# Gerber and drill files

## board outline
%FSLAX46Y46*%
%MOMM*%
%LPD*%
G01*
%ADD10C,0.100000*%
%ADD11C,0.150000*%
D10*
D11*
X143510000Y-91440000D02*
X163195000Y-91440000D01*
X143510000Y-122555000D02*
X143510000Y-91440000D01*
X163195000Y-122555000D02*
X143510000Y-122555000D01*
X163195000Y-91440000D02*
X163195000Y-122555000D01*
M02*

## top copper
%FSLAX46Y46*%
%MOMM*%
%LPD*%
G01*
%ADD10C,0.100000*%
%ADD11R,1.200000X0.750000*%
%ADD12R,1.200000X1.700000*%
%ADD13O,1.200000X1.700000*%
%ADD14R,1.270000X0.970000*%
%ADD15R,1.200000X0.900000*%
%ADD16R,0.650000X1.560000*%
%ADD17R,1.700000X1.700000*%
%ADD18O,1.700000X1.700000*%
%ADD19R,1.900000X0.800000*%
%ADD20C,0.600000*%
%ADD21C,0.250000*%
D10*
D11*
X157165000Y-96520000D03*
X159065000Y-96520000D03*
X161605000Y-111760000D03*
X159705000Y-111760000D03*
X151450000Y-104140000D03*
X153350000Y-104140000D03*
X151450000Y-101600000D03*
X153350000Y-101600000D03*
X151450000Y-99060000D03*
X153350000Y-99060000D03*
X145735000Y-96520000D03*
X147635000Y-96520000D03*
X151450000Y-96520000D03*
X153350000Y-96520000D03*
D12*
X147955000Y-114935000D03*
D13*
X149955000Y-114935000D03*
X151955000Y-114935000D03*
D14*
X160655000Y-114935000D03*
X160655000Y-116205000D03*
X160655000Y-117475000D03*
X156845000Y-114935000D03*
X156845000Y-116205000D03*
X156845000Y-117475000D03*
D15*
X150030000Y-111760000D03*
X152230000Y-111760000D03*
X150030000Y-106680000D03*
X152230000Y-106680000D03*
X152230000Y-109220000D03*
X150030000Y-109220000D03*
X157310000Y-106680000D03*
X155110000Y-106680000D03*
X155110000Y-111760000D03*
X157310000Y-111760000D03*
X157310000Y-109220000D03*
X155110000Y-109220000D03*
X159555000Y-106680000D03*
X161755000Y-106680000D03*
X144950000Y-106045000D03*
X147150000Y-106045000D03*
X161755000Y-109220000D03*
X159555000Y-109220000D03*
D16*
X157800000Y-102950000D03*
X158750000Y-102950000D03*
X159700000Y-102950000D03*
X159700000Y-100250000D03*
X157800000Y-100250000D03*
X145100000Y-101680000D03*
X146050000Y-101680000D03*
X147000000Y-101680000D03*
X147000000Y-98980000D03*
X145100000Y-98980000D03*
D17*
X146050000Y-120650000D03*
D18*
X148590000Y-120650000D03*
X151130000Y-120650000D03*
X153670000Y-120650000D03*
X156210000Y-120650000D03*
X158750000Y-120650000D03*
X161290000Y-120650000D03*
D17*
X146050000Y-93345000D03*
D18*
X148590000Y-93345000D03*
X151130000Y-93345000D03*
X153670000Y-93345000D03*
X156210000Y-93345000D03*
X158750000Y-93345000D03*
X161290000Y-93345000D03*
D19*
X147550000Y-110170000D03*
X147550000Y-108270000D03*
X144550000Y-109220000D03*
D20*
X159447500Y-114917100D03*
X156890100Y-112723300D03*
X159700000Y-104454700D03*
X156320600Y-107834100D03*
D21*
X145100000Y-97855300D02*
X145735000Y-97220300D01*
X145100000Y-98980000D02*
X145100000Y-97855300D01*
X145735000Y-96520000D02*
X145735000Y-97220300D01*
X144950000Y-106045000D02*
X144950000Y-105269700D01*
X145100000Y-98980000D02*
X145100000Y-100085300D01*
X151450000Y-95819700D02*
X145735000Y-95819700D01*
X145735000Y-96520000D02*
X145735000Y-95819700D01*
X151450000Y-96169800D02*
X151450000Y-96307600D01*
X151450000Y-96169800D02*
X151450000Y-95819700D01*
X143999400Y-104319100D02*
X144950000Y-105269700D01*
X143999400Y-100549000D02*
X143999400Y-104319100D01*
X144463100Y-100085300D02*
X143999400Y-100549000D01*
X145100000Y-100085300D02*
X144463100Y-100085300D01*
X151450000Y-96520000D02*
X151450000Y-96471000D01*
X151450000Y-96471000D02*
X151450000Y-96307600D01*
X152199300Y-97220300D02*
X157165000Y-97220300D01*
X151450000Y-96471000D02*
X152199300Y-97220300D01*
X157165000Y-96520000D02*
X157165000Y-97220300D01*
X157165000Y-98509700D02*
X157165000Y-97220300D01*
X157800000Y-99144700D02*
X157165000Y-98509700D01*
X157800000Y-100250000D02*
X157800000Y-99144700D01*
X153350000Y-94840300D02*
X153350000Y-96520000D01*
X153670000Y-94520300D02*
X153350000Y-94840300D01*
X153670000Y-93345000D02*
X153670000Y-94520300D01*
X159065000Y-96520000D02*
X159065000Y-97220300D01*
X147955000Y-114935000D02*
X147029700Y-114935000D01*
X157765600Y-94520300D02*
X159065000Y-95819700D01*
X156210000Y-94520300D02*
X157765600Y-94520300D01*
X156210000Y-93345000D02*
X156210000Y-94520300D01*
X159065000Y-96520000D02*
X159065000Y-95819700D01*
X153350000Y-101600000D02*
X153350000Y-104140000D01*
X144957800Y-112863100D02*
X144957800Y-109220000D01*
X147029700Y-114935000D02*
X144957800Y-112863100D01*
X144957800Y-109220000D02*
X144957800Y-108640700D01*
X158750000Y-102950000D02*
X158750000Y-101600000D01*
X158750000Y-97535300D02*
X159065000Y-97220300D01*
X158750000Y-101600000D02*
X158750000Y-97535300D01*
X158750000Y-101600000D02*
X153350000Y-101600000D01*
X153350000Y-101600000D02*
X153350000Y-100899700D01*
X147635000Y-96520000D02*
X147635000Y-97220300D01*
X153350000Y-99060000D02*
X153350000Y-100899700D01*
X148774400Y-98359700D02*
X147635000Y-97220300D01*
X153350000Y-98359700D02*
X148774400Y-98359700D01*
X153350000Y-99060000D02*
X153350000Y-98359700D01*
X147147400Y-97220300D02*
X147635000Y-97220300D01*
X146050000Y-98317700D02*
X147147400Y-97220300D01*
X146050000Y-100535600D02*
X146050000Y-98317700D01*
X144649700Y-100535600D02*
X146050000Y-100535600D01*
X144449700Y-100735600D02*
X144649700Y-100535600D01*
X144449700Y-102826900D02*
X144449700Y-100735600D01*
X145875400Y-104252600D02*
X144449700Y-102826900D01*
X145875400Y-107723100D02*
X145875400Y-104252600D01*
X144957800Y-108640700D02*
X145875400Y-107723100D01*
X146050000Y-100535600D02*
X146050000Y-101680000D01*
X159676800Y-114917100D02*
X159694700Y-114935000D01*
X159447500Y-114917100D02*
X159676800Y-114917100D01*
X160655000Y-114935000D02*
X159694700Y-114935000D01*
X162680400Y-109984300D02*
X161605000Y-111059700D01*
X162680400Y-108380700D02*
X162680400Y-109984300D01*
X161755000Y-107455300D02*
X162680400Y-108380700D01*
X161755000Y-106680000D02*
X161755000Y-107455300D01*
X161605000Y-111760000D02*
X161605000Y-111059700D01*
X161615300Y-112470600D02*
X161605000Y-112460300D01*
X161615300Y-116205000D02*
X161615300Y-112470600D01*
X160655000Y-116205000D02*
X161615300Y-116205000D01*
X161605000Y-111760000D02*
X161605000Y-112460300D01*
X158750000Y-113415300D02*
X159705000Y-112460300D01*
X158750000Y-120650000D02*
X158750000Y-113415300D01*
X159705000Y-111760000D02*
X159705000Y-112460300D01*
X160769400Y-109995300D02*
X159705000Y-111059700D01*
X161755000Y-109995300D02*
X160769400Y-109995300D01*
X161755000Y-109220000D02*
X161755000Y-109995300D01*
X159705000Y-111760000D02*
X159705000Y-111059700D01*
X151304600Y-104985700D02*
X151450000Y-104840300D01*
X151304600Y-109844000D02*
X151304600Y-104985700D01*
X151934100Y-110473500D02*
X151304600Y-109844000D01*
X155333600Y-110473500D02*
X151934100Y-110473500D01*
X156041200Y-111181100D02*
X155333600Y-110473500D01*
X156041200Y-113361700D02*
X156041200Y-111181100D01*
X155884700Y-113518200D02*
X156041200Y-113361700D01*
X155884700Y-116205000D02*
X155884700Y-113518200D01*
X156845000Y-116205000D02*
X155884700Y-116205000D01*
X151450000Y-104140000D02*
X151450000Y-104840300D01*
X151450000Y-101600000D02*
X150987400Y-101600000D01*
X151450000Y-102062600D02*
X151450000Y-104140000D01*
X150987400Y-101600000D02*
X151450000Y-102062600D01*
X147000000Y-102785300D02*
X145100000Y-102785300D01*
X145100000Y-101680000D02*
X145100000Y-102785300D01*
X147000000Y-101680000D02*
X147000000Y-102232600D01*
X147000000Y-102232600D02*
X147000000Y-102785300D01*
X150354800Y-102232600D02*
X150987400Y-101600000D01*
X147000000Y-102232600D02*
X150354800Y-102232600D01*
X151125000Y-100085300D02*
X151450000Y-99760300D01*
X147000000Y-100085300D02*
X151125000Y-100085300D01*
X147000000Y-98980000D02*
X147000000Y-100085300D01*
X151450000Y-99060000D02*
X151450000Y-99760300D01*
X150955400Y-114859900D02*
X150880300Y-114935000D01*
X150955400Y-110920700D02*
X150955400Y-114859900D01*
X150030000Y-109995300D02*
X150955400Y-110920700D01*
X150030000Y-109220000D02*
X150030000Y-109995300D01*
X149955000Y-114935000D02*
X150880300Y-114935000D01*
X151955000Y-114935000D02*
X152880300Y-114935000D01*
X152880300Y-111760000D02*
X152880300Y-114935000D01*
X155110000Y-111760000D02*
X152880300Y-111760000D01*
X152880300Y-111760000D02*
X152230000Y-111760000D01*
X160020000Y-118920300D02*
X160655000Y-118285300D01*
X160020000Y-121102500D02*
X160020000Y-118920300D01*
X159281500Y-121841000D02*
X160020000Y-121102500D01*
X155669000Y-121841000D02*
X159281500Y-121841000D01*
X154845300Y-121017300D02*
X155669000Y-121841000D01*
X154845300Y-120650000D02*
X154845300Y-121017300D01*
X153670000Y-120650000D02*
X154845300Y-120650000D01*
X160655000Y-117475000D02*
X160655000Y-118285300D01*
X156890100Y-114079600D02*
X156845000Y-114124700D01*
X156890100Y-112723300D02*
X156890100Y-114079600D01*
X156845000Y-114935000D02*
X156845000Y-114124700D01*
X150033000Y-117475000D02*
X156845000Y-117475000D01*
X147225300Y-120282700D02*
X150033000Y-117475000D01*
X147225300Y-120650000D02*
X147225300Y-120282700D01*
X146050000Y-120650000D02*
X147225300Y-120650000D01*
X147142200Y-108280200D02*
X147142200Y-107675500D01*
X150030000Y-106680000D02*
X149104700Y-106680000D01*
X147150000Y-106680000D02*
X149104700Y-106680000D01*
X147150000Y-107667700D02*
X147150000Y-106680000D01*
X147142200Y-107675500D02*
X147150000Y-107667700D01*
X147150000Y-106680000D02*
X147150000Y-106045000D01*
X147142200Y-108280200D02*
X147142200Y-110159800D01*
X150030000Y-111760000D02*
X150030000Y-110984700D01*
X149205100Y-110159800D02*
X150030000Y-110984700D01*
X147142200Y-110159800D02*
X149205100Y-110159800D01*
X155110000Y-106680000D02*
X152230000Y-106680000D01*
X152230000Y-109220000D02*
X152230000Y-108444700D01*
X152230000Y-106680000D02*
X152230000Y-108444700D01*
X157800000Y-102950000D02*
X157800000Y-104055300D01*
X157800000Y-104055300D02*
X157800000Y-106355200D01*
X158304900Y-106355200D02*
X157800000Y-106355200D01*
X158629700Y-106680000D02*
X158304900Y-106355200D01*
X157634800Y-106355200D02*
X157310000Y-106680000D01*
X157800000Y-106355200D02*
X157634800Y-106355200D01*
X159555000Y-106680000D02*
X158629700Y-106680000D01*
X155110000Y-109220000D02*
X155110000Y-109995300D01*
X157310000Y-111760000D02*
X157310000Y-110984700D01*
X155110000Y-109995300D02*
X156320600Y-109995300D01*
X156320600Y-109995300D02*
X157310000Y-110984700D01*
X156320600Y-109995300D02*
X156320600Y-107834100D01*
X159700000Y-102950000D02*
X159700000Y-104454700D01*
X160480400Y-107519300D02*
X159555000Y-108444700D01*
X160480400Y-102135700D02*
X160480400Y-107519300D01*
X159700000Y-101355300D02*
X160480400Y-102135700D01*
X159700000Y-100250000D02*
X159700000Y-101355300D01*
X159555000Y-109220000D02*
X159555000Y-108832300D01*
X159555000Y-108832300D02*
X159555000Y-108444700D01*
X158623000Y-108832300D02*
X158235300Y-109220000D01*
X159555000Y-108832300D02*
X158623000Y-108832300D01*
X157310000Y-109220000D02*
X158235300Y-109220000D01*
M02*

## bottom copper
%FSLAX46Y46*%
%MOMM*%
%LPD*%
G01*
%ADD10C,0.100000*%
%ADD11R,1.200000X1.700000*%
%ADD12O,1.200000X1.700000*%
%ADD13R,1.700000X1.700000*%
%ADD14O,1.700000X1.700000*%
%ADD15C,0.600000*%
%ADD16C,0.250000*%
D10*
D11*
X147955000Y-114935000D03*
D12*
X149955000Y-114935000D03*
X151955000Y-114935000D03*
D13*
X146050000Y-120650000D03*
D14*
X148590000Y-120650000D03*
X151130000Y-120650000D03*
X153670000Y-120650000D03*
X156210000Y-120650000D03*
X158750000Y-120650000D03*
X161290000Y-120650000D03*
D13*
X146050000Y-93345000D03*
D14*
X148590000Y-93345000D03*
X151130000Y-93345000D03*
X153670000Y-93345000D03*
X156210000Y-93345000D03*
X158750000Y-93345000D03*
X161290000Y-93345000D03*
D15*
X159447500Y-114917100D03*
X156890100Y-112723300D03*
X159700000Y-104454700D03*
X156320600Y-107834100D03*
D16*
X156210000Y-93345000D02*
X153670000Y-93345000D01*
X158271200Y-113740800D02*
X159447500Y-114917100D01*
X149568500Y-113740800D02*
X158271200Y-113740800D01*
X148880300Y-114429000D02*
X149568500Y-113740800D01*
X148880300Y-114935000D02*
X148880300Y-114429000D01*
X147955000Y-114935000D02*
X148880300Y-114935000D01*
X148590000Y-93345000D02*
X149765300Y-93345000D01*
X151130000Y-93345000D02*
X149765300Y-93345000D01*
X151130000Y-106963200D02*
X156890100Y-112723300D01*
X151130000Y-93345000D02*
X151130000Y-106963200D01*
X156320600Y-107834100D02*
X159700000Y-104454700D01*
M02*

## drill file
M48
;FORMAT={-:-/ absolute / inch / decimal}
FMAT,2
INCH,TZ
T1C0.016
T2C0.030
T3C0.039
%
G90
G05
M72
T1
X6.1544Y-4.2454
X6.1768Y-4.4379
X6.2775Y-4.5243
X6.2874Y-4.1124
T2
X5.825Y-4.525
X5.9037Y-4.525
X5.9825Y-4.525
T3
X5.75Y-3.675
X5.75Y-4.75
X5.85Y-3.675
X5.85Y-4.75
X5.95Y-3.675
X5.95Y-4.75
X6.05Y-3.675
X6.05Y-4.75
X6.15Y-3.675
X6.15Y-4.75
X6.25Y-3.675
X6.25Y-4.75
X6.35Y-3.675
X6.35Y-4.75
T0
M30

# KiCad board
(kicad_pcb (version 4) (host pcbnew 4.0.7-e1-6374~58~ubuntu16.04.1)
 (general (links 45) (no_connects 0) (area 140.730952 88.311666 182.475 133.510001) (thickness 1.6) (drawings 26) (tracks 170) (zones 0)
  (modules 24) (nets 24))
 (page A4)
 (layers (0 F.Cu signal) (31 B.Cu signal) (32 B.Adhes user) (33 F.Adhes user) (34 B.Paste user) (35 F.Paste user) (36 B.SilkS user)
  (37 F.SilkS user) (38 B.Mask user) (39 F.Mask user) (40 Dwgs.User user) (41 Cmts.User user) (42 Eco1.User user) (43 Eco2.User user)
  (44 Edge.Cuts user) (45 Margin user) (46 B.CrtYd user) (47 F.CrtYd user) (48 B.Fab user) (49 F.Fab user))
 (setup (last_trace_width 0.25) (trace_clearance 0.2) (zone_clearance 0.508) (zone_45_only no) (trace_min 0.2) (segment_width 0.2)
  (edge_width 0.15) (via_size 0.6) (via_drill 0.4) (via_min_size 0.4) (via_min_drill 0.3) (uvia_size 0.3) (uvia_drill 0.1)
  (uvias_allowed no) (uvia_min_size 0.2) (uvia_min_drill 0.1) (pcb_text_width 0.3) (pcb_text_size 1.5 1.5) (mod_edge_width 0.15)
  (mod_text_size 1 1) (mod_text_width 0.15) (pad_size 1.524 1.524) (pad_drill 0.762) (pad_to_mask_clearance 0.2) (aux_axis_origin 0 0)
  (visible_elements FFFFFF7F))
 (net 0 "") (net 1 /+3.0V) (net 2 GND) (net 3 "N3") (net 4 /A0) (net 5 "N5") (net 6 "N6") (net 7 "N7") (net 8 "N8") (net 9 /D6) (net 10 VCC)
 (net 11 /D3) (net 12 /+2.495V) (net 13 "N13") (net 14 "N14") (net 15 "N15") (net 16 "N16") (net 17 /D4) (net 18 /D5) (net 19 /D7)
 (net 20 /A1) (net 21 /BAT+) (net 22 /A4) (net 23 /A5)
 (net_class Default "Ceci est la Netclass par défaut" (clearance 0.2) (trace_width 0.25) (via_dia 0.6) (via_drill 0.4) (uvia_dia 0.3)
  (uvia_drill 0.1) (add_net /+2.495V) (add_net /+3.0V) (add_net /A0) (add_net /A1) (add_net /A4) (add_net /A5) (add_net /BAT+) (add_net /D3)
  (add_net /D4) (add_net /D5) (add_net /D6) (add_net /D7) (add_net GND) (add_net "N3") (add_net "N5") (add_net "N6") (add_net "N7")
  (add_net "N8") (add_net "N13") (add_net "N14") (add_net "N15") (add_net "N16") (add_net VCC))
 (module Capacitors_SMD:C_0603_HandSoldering (layer F.Cu) (at 158.115 96.52)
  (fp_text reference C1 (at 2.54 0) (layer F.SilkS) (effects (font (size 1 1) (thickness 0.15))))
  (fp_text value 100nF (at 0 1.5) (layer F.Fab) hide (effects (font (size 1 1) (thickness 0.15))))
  (pad 1 smd rect (at -0.95 0) (size 1.2 0.75) (layers F.Cu F.Paste F.Mask) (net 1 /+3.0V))
  (pad 2 smd rect (at 0.95 0) (size 1.2 0.75) (layers F.Cu F.Paste F.Mask) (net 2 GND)))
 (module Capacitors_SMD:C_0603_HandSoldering (layer F.Cu) (at 160.655 111.76 180)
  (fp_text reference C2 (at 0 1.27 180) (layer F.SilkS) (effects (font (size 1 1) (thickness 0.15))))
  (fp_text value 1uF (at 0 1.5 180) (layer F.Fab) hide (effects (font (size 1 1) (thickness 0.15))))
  (pad 1 smd rect (at -0.95 0 180) (size 1.2 0.75) (layers F.Cu F.Paste F.Mask) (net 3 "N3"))
  (pad 2 smd rect (at 0.95 0 180) (size 1.2 0.75) (layers F.Cu F.Paste F.Mask) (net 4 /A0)))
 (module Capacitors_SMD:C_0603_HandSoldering (layer F.Cu) (at 152.4 104.14)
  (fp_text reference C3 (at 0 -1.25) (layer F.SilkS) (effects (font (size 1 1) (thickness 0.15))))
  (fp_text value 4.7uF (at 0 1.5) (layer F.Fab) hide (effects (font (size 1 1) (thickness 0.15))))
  (pad 1 smd rect (at -0.95 0) (size 1.2 0.75) (layers F.Cu F.Paste F.Mask) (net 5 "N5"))
  (pad 2 smd rect (at 0.95 0) (size 1.2 0.75) (layers F.Cu F.Paste F.Mask) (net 2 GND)))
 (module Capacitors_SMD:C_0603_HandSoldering (layer F.Cu) (at 152.4 101.6)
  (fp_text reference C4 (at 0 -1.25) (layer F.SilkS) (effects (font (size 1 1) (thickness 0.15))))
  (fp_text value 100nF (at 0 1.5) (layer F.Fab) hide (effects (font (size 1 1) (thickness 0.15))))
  (pad 1 smd rect (at -0.95 0) (size 1.2 0.75) (layers F.Cu F.Paste F.Mask) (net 5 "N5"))
  (pad 2 smd rect (at 0.95 0) (size 1.2 0.75) (layers F.Cu F.Paste F.Mask) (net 2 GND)))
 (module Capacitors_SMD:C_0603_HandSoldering (layer F.Cu) (at 152.4 99.06)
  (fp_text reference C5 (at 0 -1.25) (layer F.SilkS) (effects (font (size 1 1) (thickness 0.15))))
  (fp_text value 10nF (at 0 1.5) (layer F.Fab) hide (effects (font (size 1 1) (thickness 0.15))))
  (pad 1 smd rect (at -0.95 0) (size 1.2 0.75) (layers F.Cu F.Paste F.Mask) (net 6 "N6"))
  (pad 2 smd rect (at 0.95 0) (size 1.2 0.75) (layers F.Cu F.Paste F.Mask) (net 2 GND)))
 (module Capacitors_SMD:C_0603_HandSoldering (layer F.Cu) (at 146.685 96.52)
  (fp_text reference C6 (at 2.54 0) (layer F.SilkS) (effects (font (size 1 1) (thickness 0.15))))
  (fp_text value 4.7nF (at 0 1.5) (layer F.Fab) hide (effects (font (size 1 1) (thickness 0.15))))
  (pad 1 smd rect (at -0.95 0) (size 1.2 0.75) (layers F.Cu F.Paste F.Mask) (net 1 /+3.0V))
  (pad 2 smd rect (at 0.95 0) (size 1.2 0.75) (layers F.Cu F.Paste F.Mask) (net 2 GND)))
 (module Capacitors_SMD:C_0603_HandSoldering (layer F.Cu) (at 152.4 96.52)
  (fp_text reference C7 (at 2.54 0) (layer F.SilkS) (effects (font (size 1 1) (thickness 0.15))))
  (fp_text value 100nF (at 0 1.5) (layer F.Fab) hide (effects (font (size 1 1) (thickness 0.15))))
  (pad 1 smd rect (at -0.95 0) (size 1.2 0.75) (layers F.Cu F.Paste F.Mask) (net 1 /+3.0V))
  (pad 2 smd rect (at 0.95 0) (size 1.2 0.75) (layers F.Cu F.Paste F.Mask) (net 2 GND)))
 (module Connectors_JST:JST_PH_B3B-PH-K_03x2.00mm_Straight (layer F.Cu) (at 147.955 114.935)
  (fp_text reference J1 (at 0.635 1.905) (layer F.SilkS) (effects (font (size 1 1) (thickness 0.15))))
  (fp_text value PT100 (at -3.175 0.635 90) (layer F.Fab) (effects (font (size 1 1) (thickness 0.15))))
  (pad 1 thru_hole rect (at 0 0) (size 1.2 1.7) (drill 0.75) (layers *.Cu *.Mask) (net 2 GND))
  (pad 2 thru_hole oval (at 2 0) (size 1.2 1.7) (drill 0.75) (layers *.Cu *.Mask) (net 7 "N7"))
  (pad 3 thru_hole oval (at 4 0) (size 1.2 1.7) (drill 0.75) (layers *.Cu *.Mask) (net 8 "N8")))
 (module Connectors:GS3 (layer F.Cu) (at 160.655 116.205)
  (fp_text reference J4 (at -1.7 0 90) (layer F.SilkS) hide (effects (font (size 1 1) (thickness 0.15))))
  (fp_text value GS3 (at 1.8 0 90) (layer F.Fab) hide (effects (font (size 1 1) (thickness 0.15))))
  (pad 1 smd rect (at 0 -1.27) (size 1.27 0.97) (layers F.Cu F.Paste F.Mask) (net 2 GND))
  (pad 2 smd rect (at 0 0) (size 1.27 0.97) (layers F.Cu F.Paste F.Mask) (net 3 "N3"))
  (pad 3 smd rect (at 0 1.27) (size 1.27 0.97) (layers F.Cu F.Paste F.Mask) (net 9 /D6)))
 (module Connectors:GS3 (layer F.Cu) (at 156.845 116.205)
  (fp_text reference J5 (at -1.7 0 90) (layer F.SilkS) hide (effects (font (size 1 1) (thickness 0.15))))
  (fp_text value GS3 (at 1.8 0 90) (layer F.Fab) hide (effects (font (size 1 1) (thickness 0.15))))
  (pad 1 smd rect (at 0 -1.27) (size 1.27 0.97) (layers F.Cu F.Paste F.Mask) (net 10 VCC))
  (pad 2 smd rect (at 0 0) (size 1.27 0.97) (layers F.Cu F.Paste F.Mask) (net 5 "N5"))
  (pad 3 smd rect (at 0 1.27) (size 1.27 0.97) (layers F.Cu F.Paste F.Mask) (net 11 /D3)))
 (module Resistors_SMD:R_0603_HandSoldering (layer F.Cu) (at 151.13 111.76)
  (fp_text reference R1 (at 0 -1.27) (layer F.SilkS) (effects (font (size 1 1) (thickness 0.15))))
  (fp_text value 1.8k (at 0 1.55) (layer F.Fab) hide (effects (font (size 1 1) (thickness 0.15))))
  (pad 1 smd rect (at -1.1 0) (size 1.2 0.9) (layers F.Cu F.Paste F.Mask) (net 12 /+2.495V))
  (pad 2 smd rect (at 1.1 0) (size 1.2 0.9) (layers F.Cu F.Paste F.Mask) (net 8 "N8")))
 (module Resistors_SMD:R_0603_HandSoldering (layer F.Cu) (at 151.13 106.68)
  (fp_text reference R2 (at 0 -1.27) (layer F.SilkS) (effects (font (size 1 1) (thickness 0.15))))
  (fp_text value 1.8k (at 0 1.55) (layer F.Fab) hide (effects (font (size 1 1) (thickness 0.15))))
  (pad 1 smd rect (at -1.1 0) (size 1.2 0.9) (layers F.Cu F.Paste F.Mask) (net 12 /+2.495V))
  (pad 2 smd rect (at 1.1 0) (size 1.2 0.9) (layers F.Cu F.Paste F.Mask) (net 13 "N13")))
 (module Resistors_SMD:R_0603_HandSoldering (layer F.Cu) (at 151.13 109.22 180)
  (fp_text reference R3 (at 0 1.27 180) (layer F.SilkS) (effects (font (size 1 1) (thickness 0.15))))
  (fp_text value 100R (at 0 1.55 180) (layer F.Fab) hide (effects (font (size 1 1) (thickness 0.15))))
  (pad 1 smd rect (at -1.1 0 180) (size 1.2 0.9) (layers F.Cu F.Paste F.Mask) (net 13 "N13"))
  (pad 2 smd rect (at 1.1 0 180) (size 1.2 0.9) (layers F.Cu F.Paste F.Mask) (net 7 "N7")))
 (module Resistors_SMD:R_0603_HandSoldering (layer F.Cu) (at 156.21 106.68 180)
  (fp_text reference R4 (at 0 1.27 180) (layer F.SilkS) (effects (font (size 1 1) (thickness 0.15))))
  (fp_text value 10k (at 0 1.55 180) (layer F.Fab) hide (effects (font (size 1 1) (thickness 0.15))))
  (pad 1 smd rect (at -1.1 0 180) (size 1.2 0.9) (layers F.Cu F.Paste F.Mask) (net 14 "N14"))
  (pad 2 smd rect (at 1.1 0 180) (size 1.2 0.9) (layers F.Cu F.Paste F.Mask) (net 13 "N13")))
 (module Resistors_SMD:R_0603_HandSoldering (layer F.Cu) (at 156.21 111.76)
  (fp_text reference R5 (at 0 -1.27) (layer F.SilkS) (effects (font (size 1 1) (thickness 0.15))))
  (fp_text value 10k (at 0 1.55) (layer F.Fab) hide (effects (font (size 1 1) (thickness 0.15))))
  (pad 1 smd rect (at -1.1 0) (size 1.2 0.9) (layers F.Cu F.Paste F.Mask) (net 8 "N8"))
  (pad 2 smd rect (at 1.1 0) (size 1.2 0.9) (layers F.Cu F.Paste F.Mask) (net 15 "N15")))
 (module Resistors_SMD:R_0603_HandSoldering (layer F.Cu) (at 156.21 109.22 180)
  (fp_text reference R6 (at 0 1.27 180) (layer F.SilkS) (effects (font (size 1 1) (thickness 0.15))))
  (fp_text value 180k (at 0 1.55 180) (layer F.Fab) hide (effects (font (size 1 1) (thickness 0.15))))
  (pad 1 smd rect (at -1.1 0 180) (size 1.2 0.9) (layers F.Cu F.Paste F.Mask) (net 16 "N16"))
  (pad 2 smd rect (at 1.1 0 180) (size 1.2 0.9) (layers F.Cu F.Paste F.Mask) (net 15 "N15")))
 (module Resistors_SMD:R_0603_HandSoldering (layer F.Cu) (at 160.655 106.68)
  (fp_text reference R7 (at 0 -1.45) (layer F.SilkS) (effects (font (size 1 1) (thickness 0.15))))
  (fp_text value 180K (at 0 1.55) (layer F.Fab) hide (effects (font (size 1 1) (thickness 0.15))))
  (pad 1 smd rect (at -1.1 0) (size 1.2 0.9) (layers F.Cu F.Paste F.Mask) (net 14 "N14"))
  (pad 2 smd rect (at 1.1 0) (size 1.2 0.9) (layers F.Cu F.Paste F.Mask) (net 3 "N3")))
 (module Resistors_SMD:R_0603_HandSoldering (layer F.Cu) (at 146.05 106.045)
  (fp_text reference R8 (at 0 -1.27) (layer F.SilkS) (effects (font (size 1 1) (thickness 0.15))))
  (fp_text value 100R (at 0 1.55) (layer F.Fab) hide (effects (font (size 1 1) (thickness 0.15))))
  (pad 1 smd rect (at -1.1 0) (size 1.2 0.9) (layers F.Cu F.Paste F.Mask) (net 1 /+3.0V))
  (pad 2 smd rect (at 1.1 0) (size 1.2 0.9) (layers F.Cu F.Paste F.Mask) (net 12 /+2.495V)))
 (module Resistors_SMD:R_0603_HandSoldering (layer F.Cu) (at 160.655 109.22 180)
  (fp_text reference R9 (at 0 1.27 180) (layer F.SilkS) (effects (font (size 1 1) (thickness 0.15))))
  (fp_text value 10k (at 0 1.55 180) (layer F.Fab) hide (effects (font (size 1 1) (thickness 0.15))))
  (pad 1 smd rect (at -1.1 0 180) (size 1.2 0.9) (layers F.Cu F.Paste F.Mask) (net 4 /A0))
  (pad 2 smd rect (at 1.1 0 180) (size 1.2 0.9) (layers F.Cu F.Paste F.Mask) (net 16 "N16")))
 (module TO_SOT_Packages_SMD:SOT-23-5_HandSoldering (layer F.Cu) (at 158.75 101.6 90)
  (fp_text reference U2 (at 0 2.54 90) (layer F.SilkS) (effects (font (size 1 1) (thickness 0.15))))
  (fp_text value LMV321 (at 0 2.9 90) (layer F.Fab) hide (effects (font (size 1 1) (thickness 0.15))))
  (pad 1 smd rect (at -1.35 -0.95 90) (size 1.56 0.65) (layers F.Cu F.Paste F.Mask) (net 14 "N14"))
  (pad 2 smd rect (at -1.35 0 90) (size 1.56 0.65) (layers F.Cu F.Paste F.Mask) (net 2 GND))
  (pad 3 smd rect (at -1.35 0.95 90) (size 1.56 0.65) (layers F.Cu F.Paste F.Mask) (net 15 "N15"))
  (pad 4 smd rect (at 1.35 0.95 90) (size 1.56 0.65) (layers F.Cu F.Paste F.Mask) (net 16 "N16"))
  (pad 5 smd rect (at 1.35 -0.95 90) (size 1.56 0.65) (layers F.Cu F.Paste F.Mask) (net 1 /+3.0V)))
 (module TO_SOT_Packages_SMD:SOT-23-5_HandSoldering (layer F.Cu) (at 146.05 100.33 90)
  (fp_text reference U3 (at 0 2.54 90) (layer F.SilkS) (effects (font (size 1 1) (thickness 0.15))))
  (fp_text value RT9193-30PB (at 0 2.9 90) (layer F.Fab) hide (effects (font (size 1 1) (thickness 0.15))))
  (pad 1 smd rect (at -1.35 -0.95 90) (size 1.56 0.65) (layers F.Cu F.Paste F.Mask) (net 5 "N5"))
  (pad 2 smd rect (at -1.35 0 90) (size 1.56 0.65) (layers F.Cu F.Paste F.Mask) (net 2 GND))
  (pad 3 smd rect (at -1.35 0.95 90) (size 1.56 0.65) (layers F.Cu F.Paste F.Mask) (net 5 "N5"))
  (pad 4 smd rect (at 1.35 0.95 90) (size 1.56 0.65) (layers F.Cu F.Paste F.Mask) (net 6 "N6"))
  (pad 5 smd rect (at 1.35 -0.95 90) (size 1.56 0.65) (layers F.Cu F.Paste F.Mask) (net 1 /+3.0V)))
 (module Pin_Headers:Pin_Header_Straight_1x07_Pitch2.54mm (layer B.Cu) (at 146.05 120.65 270)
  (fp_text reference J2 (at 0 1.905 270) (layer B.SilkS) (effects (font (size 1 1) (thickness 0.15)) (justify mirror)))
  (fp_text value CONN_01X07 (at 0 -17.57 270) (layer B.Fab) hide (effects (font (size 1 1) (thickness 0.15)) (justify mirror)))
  (pad 1 thru_hole rect (at 0 0 270) (size 1.7 1.7) (drill 1) (layers *.Cu *.Mask) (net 11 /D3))
  (pad 2 thru_hole oval (at 0 -2.54 270) (size 1.7 1.7) (drill 1) (layers *.Cu *.Mask) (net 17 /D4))
  (pad 3 thru_hole oval (at 0 -5.08 270) (size 1.7 1.7) (drill 1) (layers *.Cu *.Mask) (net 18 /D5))
  (pad 4 thru_hole oval (at 0 -7.62 270) (size 1.7 1.7) (drill 1) (layers *.Cu *.Mask) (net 9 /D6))
  (pad 5 thru_hole oval (at 0 -10.16 270) (size 1.7 1.7) (drill 1) (layers *.Cu *.Mask) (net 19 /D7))
  (pad 6 thru_hole oval (at 0 -12.7 270) (size 1.7 1.7) (drill 1) (layers *.Cu *.Mask) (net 4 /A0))
  (pad 7 thru_hole oval (at 0 -15.24 270) (size 1.7 1.7) (drill 1) (layers *.Cu *.Mask) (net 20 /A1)))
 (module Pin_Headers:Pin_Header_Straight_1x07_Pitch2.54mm (layer B.Cu) (at 146.05 93.345 270)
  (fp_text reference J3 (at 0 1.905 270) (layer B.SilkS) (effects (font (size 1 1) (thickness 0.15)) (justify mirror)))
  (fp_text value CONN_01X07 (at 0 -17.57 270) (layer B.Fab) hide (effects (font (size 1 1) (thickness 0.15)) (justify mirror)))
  (pad 1 thru_hole rect (at 0 0 270) (size 1.7 1.7) (drill 1) (layers *.Cu *.Mask) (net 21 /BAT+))
  (pad 2 thru_hole oval (at 0 -2.54 270) (size 1.7 1.7) (drill 1) (layers *.Cu *.Mask) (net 10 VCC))
  (pad 3 thru_hole oval (at 0 -5.08 270) (size 1.7 1.7) (drill 1) (layers *.Cu *.Mask) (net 10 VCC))
  (pad 4 thru_hole oval (at 0 -7.62 270) (size 1.7 1.7) (drill 1) (layers *.Cu *.Mask) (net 2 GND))
  (pad 5 thru_hole oval (at 0 -10.16 270) (size 1.7 1.7) (drill 1) (layers *.Cu *.Mask) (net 2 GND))
  (pad 6 thru_hole oval (at 0 -12.7 270) (size 1.7 1.7) (drill 1) (layers *.Cu *.Mask) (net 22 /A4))
  (pad 7 thru_hole oval (at 0 -15.24 270) (size 1.7 1.7) (drill 1) (layers *.Cu *.Mask) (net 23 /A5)))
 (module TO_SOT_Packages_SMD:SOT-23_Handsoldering (layer F.Cu) (at 146.05 109.22 180)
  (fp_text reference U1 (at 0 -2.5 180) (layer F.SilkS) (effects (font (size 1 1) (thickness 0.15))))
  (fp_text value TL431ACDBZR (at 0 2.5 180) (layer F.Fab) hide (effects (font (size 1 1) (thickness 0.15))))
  (pad 1 smd rect (at -1.5 -0.95 180) (size 1.9 0.8) (layers F.Cu F.Paste F.Mask) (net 12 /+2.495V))
  (pad 2 smd rect (at -1.5 0.95 180) (size 1.9 0.8) (layers F.Cu F.Paste F.Mask) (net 12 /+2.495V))
  (pad 3 smd rect (at 1.5 0 180) (size 1.9 0.8) (layers F.Cu F.Paste F.Mask) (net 2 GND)))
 (gr_line (start 143.51 91.44) (end 163.195 91.44) (angle 90) (layer Edge.Cuts) (width 0.15))
 (gr_line (start 143.51 122.555) (end 143.51 91.44) (angle 90) (layer Edge.Cuts) (width 0.15))
 (gr_line (start 163.195 122.555) (end 143.51 122.555) (angle 90) (layer Edge.Cuts) (width 0.15))
 (gr_line (start 163.195 91.44) (end 163.195 122.555) (angle 90) (layer Edge.Cuts) (width 0.15))
 (segment (start 145.1 97.8553) (end 145.735 97.2203) (width 0.25) (layer F.Cu) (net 1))
 (segment (start 145.1 98.98) (end 145.1 97.8553) (width 0.25) (layer F.Cu) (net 1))
 (segment (start 145.735 96.52) (end 145.735 97.2203) (width 0.25) (layer F.Cu) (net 1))
 (segment (start 144.95 106.045) (end 144.95 105.2697) (width 0.25) (layer F.Cu) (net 1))
 (segment (start 145.1 98.98) (end 145.1 100.0853) (width 0.25) (layer F.Cu) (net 1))
 (segment (start 151.45 95.8197) (end 145.735 95.8197) (width 0.25) (layer F.Cu) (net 1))
 (segment (start 145.735 96.52) (end 145.735 95.8197) (width 0.25) (layer F.Cu) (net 1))
 (segment (start 151.45 96.1698) (end 151.45 96.3076) (width 0.25) (layer F.Cu) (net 1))
 (segment (start 151.45 96.1698) (end 151.45 95.8197) (width 0.25) (layer F.Cu) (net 1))
 (segment (start 143.9994 104.3191) (end 144.95 105.2697) (width 0.25) (layer F.Cu) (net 1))
 (segment (start 143.9994 100.549) (end 143.9994 104.3191) (width 0.25) (layer F.Cu) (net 1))
 (segment (start 144.4631 100.0853) (end 143.9994 100.549) (width 0.25) (layer F.Cu) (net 1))
 (segment (start 145.1 100.0853) (end 144.4631 100.0853) (width 0.25) (layer F.Cu) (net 1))
 (segment (start 151.45 96.52) (end 151.45 96.471) (width 0.25) (layer F.Cu) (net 1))
 (segment (start 151.45 96.471) (end 151.45 96.3076) (width 0.25) (layer F.Cu) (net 1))
 (segment (start 152.1993 97.2203) (end 157.165 97.2203) (width 0.25) (layer F.Cu) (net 1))
 (segment (start 151.45 96.471) (end 152.1993 97.2203) (width 0.25) (layer F.Cu) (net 1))
 (segment (start 157.165 96.52) (end 157.165 97.2203) (width 0.25) (layer F.Cu) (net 1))
 (segment (start 157.165 98.5097) (end 157.165 97.2203) (width 0.25) (layer F.Cu) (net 1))
 (segment (start 157.8 99.1447) (end 157.165 98.5097) (width 0.25) (layer F.Cu) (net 1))
 (segment (start 157.8 100.25) (end 157.8 99.1447) (width 0.25) (layer F.Cu) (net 1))
 (via (at 159.4475 114.9171) (size 0.6) (layers F.Cu B.Cu) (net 2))
 (segment (start 156.21 93.345) (end 153.67 93.345) (width 0.25) (layer B.Cu) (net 2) (status 30))
 (segment (start 153.35 94.8403) (end 153.35 96.52) (width 0.25) (layer F.Cu) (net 2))
 (segment (start 153.67 94.5203) (end 153.35 94.8403) (width 0.25) (layer F.Cu) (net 2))
 (segment (start 153.67 93.345) (end 153.67 94.5203) (width 0.25) (layer F.Cu) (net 2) (status 10))
 (segment (start 159.065 96.52) (end 159.065 97.2203) (width 0.25) (layer F.Cu) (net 2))
 (segment (start 147.955 114.935) (end 147.0297 114.935) (width 0.25) (layer F.Cu) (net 2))
 (segment (start 157.7656 94.5203) (end 159.065 95.8197) (width 0.25) (layer F.Cu) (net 2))
 (segment (start 156.21 94.5203) (end 157.7656 94.5203) (width 0.25) (layer F.Cu) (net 2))
 (segment (start 156.21 93.345) (end 156.21 94.5203) (width 0.25) (layer F.Cu) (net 2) (status 10))
 (segment (start 159.065 96.52) (end 159.065 95.8197) (width 0.25) (layer F.Cu) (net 2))
 (segment (start 153.35 101.6) (end 153.35 104.14) (width 0.25) (layer F.Cu) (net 2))
 (segment (start 144.9578 112.8631) (end 144.9578 109.22) (width 0.25) (layer F.Cu) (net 2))
 (segment (start 147.0297 114.935) (end 144.9578 112.8631) (width 0.25) (layer F.Cu) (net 2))
 (segment (start 144.9578 109.22) (end 144.9578 108.6407) (width 0.25) (layer F.Cu) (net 2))
 (segment (start 158.75 102.95) (end 158.75 101.6) (width 0.25) (layer F.Cu) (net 2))
 (segment (start 158.75 97.5353) (end 159.065 97.2203) (width 0.25) (layer F.Cu) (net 2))
 (segment (start 158.75 101.6) (end 158.75 97.5353) (width 0.25) (layer F.Cu) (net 2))
 (segment (start 158.75 101.6) (end 153.35 101.6) (width 0.25) (layer F.Cu) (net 2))
 (segment (start 153.35 101.6) (end 153.35 100.8997) (width 0.25) (layer F.Cu) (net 2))
 (segment (start 147.635 96.52) (end 147.635 97.2203) (width 0.25) (layer F.Cu) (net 2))
 (segment (start 153.35 99.06) (end 153.35 100.8997) (width 0.25) (layer F.Cu) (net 2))
 (segment (start 148.7744 98.3597) (end 147.635 97.2203) (width 0.25) (layer F.Cu) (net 2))
 (segment (start 153.35 98.3597) (end 148.7744 98.3597) (width 0.25) (layer F.Cu) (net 2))
 (segment (start 153.35 99.06) (end 153.35 98.3597) (width 0.25) (layer F.Cu) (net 2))
 (segment (start 147.1474 97.2203) (end 147.635 97.2203) (width 0.25) (layer F.Cu) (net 2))
 (segment (start 146.05 98.3177) (end 147.1474 97.2203) (width 0.25) (layer F.Cu) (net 2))
 (segment (start 146.05 100.5356) (end 146.05 98.3177) (width 0.25) (layer F.Cu) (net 2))
 (segment (start 144.6497 100.5356) (end 146.05 100.5356) (width 0.25) (layer F.Cu) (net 2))
 (segment (start 144.4497 100.7356) (end 144.6497 100.5356) (width 0.25) (layer F.Cu) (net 2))
 (segment (start 144.4497 102.8269) (end 144.4497 100.7356) (width 0.25) (layer F.Cu) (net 2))
 (segment (start 145.8754 104.2526) (end 144.4497 102.8269) (width 0.25) (layer F.Cu) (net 2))
 (segment (start 145.8754 107.7231) (end 145.8754 104.2526) (width 0.25) (layer F.Cu) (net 2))
 (segment (start 144.9578 108.6407) (end 145.8754 107.7231) (width 0.25) (layer F.Cu) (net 2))
 (segment (start 146.05 100.5356) (end 146.05 101.68) (width 0.25) (layer F.Cu) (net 2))
 (segment (start 158.2712 113.7408) (end 159.4475 114.9171) (width 0.25) (layer B.Cu) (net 2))
 (segment (start 149.5685 113.7408) (end 158.2712 113.7408) (width 0.25) (layer B.Cu) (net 2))
 (segment (start 148.8803 114.429) (end 149.5685 113.7408) (width 0.25) (layer B.Cu) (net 2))
 (segment (start 148.8803 114.935) (end 148.8803 114.429) (width 0.25) (layer B.Cu) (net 2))
 (segment (start 159.6768 114.9171) (end 159.6947 114.935) (width 0.25) (layer F.Cu) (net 2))
 (segment (start 159.4475 114.9171) (end 159.6768 114.9171) (width 0.25) (layer F.Cu) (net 2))
 (segment (start 160.655 114.935) (end 159.6947 114.935) (width 0.25) (layer F.Cu) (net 2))
 (segment (start 147.955 114.935) (end 148.8803 114.935) (width 0.25) (layer B.Cu) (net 2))
 (segment (start 162.6804 109.9843) (end 161.605 111.0597) (width 0.25) (layer F.Cu) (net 3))
 (segment (start 162.6804 108.3807) (end 162.6804 109.9843) (width 0.25) (layer F.Cu) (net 3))
 (segment (start 161.755 107.4553) (end 162.6804 108.3807) (width 0.25) (layer F.Cu) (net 3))
 (segment (start 161.755 106.68) (end 161.755 107.4553) (width 0.25) (layer F.Cu) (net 3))
 (segment (start 161.605 111.76) (end 161.605 111.0597) (width 0.25) (layer F.Cu) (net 3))
 (segment (start 161.6153 112.4706) (end 161.605 112.4603) (width 0.25) (layer F.Cu) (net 3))
 (segment (start 161.6153 116.205) (end 161.6153 112.4706) (width 0.25) (layer F.Cu) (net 3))
 (segment (start 160.655 116.205) (end 161.6153 116.205) (width 0.25) (layer F.Cu) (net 3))
 (segment (start 161.605 111.76) (end 161.605 112.4603) (width 0.25) (layer F.Cu) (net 3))
 (segment (start 158.75 113.4153) (end 159.705 112.4603) (width 0.25) (layer F.Cu) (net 4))
 (segment (start 158.75 120.65) (end 158.75 113.4153) (width 0.25) (layer F.Cu) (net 4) (status 10))
 (segment (start 159.705 111.76) (end 159.705 112.4603) (width 0.25) (layer F.Cu) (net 4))
 (segment (start 160.7694 109.9953) (end 159.705 111.0597) (width 0.25) (layer F.Cu) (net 4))
 (segment (start 161.755 109.9953) (end 160.7694 109.9953) (width 0.25) (layer F.Cu) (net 4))
 (segment (start 161.755 109.22) (end 161.755 109.9953) (width 0.25) (layer F.Cu) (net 4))
 (segment (start 159.705 111.76) (end 159.705 111.0597) (width 0.25) (layer F.Cu) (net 4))
 (segment (start 151.3046 104.9857) (end 151.45 104.8403) (width 0.25) (layer F.Cu) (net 5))
 (segment (start 151.3046 109.844) (end 151.3046 104.9857) (width 0.25) (layer F.Cu) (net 5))
 (segment (start 151.9341 110.4735) (end 151.3046 109.844) (width 0.25) (layer F.Cu) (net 5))
 (segment (start 155.3336 110.4735) (end 151.9341 110.4735) (width 0.25) (layer F.Cu) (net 5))
 (segment (start 156.0412 111.1811) (end 155.3336 110.4735) (width 0.25) (layer F.Cu) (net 5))
 (segment (start 156.0412 113.3617) (end 156.0412 111.1811) (width 0.25) (layer F.Cu) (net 5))
 (segment (start 155.8847 113.5182) (end 156.0412 113.3617) (width 0.25) (layer F.Cu) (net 5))
 (segment (start 155.8847 116.205) (end 155.8847 113.5182) (width 0.25) (layer F.Cu) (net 5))
 (segment (start 156.845 116.205) (end 155.8847 116.205) (width 0.25) (layer F.Cu) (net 5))
 (segment (start 151.45 104.14) (end 151.45 104.8403) (width 0.25) (layer F.Cu) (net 5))
 (segment (start 151.45 101.6) (end 150.9874 101.6) (width 0.25) (layer F.Cu) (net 5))
 (segment (start 151.45 102.0626) (end 151.45 104.14) (width 0.25) (layer F.Cu) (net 5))
 (segment (start 150.9874 101.6) (end 151.45 102.0626) (width 0.25) (layer F.Cu) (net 5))
 (segment (start 147 102.7853) (end 145.1 102.7853) (width 0.25) (layer F.Cu) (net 5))
 (segment (start 145.1 101.68) (end 145.1 102.7853) (width 0.25) (layer F.Cu) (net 5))
 (segment (start 147 101.68) (end 147 102.2326) (width 0.25) (layer F.Cu) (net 5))
 (segment (start 147 102.2326) (end 147 102.7853) (width 0.25) (layer F.Cu) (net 5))
 (segment (start 150.3548 102.2326) (end 150.9874 101.6) (width 0.25) (layer F.Cu) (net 5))
 (segment (start 147 102.2326) (end 150.3548 102.2326) (width 0.25) (layer F.Cu) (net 5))
 (segment (start 151.125 100.0853) (end 151.45 99.7603) (width 0.25) (layer F.Cu) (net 6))
 (segment (start 147 100.0853) (end 151.125 100.0853) (width 0.25) (layer F.Cu) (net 6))
 (segment (start 147 98.98) (end 147 100.0853) (width 0.25) (layer F.Cu) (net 6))
 (segment (start 151.45 99.06) (end 151.45 99.7603) (width 0.25) (layer F.Cu) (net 6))
 (segment (start 150.9554 114.8599) (end 150.8803 114.935) (width 0.25) (layer F.Cu) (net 7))
 (segment (start 150.9554 110.9207) (end 150.9554 114.8599) (width 0.25) (layer F.Cu) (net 7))
 (segment (start 150.03 109.9953) (end 150.9554 110.9207) (width 0.25) (layer F.Cu) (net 7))
 (segment (start 150.03 109.22) (end 150.03 109.9953) (width 0.25) (layer F.Cu) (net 7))
 (segment (start 149.955 114.935) (end 150.8803 114.935) (width 0.25) (layer F.Cu) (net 7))
 (segment (start 151.955 114.935) (end 152.8803 114.935) (width 0.25) (layer F.Cu) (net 8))
 (segment (start 152.8803 111.76) (end 152.8803 114.935) (width 0.25) (layer F.Cu) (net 8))
 (segment (start 155.11 111.76) (end 152.8803 111.76) (width 0.25) (layer F.Cu) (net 8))
 (segment (start 152.8803 111.76) (end 152.23 111.76) (width 0.25) (layer F.Cu) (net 8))
 (segment (start 160.02 118.9203) (end 160.655 118.2853) (width 0.25) (layer F.Cu) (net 9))
 (segment (start 160.02 121.1025) (end 160.02 118.9203) (width 0.25) (layer F.Cu) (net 9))
 (segment (start 159.2815 121.841) (end 160.02 121.1025) (width 0.25) (layer F.Cu) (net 9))
 (segment (start 155.669 121.841) (end 159.2815 121.841) (width 0.25) (layer F.Cu) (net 9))
 (segment (start 154.8453 121.0173) (end 155.669 121.841) (width 0.25) (layer F.Cu) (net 9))
 (segment (start 154.8453 120.65) (end 154.8453 121.0173) (width 0.25) (layer F.Cu) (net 9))
 (segment (start 153.67 120.65) (end 154.8453 120.65) (width 0.25) (layer F.Cu) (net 9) (status 10))
 (segment (start 160.655 117.475) (end 160.655 118.2853) (width 0.25) (layer F.Cu) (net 9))
 (via (at 156.8901 112.7233) (size 0.6) (layers F.Cu B.Cu) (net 10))
 (segment (start 148.59 93.345) (end 149.7653 93.345) (width 0.25) (layer B.Cu) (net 10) (status 10))
 (segment (start 151.13 93.345) (end 149.7653 93.345) (width 0.25) (layer B.Cu) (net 10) (status 10))
 (segment (start 156.8901 114.0796) (end 156.845 114.1247) (width 0.25) (layer F.Cu) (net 10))
 (segment (start 156.8901 112.7233) (end 156.8901 114.0796) (width 0.25) (layer F.Cu) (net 10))
 (segment (start 156.845 114.935) (end 156.845 114.1247) (width 0.25) (layer F.Cu) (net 10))
 (segment (start 151.13 106.9632) (end 156.8901 112.7233) (width 0.25) (layer B.Cu) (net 10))
 (segment (start 151.13 93.345) (end 151.13 106.9632) (width 0.25) (layer B.Cu) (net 10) (status 10))
 (segment (start 150.033 117.475) (end 156.845 117.475) (width 0.25) (layer F.Cu) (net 11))
 (segment (start 147.2253 120.2827) (end 150.033 117.475) (width 0.25) (layer F.Cu) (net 11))
 (segment (start 147.2253 120.65) (end 147.2253 120.2827) (width 0.25) (layer F.Cu) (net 11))
 (segment (start 146.05 120.65) (end 147.2253 120.65) (width 0.25) (layer F.Cu) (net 11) (status 10))
 (segment (start 147.1422 108.2802) (end 147.1422 107.6755) (width 0.25) (layer F.Cu) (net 12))
 (segment (start 150.03 106.68) (end 149.1047 106.68) (width 0.25) (layer F.Cu) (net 12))
 (segment (start 147.15 106.68) (end 149.1047 106.68) (width 0.25) (layer F.Cu) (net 12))
 (segment (start 147.15 107.6677) (end 147.15 106.68) (width 0.25) (layer F.Cu) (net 12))
 (segment (start 147.1422 107.6755) (end 147.15 107.6677) (width 0.25) (layer F.Cu) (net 12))
 (segment (start 147.15 106.68) (end 147.15 106.045) (width 0.25) (layer F.Cu) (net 12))
 (segment (start 147.1422 108.2802) (end 147.1422 110.1598) (width 0.25) (layer F.Cu) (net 12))
 (segment (start 150.03 111.76) (end 150.03 110.9847) (width 0.25) (layer F.Cu) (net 12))
 (segment (start 149.2051 110.1598) (end 150.03 110.9847) (width 0.25) (layer F.Cu) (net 12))
 (segment (start 147.1422 110.1598) (end 149.2051 110.1598) (width 0.25) (layer F.Cu) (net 12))
 (segment (start 155.11 106.68) (end 152.23 106.68) (width 0.25) (layer F.Cu) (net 13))
 (segment (start 152.23 109.22) (end 152.23 108.4447) (width 0.25) (layer F.Cu) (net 13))
 (segment (start 152.23 106.68) (end 152.23 108.4447) (width 0.25) (layer F.Cu) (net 13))
 (segment (start 157.8 102.95) (end 157.8 104.0553) (width 0.25) (layer F.Cu) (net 14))
 (segment (start 157.8 104.0553) (end 157.8 106.3552) (width 0.25) (layer F.Cu) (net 14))
 (segment (start 158.3049 106.3552) (end 157.8 106.3552) (width 0.25) (layer F.Cu) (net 14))
 (segment (start 158.6297 106.68) (end 158.3049 106.3552) (width 0.25) (layer F.Cu) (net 14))
 (segment (start 157.6348 106.3552) (end 157.31 106.68) (width 0.25) (layer F.Cu) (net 14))
 (segment (start 157.8 106.3552) (end 157.6348 106.3552) (width 0.25) (layer F.Cu) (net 14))
 (segment (start 159.555 106.68) (end 158.6297 106.68) (width 0.25) (layer F.Cu) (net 14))
 (via (at 159.7 104.4547) (size 0.6) (layers F.Cu B.Cu) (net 15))
 (via (at 156.3206 107.8341) (size 0.6) (layers F.Cu B.Cu) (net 15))
 (segment (start 155.11 109.22) (end 155.11 109.9953) (width 0.25) (layer F.Cu) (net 15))
 (segment (start 157.31 111.76) (end 157.31 110.9847) (width 0.25) (layer F.Cu) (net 15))
 (segment (start 155.11 109.9953) (end 156.3206 109.9953) (width 0.25) (layer F.Cu) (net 15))
 (segment (start 156.3206 109.9953) (end 157.31 110.9847) (width 0.25) (layer F.Cu) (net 15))
 (segment (start 156.3206 109.9953) (end 156.3206 107.8341) (width 0.25) (layer F.Cu) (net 15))
 (segment (start 156.3206 107.8341) (end 159.7 104.4547) (width 0.25) (layer B.Cu) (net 15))
 (segment (start 159.7 102.95) (end 159.7 104.4547) (width 0.25) (layer F.Cu) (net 15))
 (segment (start 160.4804 107.5193) (end 159.555 108.4447) (width 0.25) (layer F.Cu) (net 16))
 (segment (start 160.4804 102.1357) (end 160.4804 107.5193) (width 0.25) (layer F.Cu) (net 16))
 (segment (start 159.7 101.3553) (end 160.4804 102.1357) (width 0.25) (layer F.Cu) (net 16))
 (segment (start 159.7 100.25) (end 159.7 101.3553) (width 0.25) (layer F.Cu) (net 16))
 (segment (start 159.555 109.22) (end 159.555 108.8323) (width 0.25) (layer F.Cu) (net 16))
 (segment (start 159.555 108.8323) (end 159.555 108.4447) (width 0.25) (layer F.Cu) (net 16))
 (segment (start 158.623 108.8323) (end 158.2353 109.22) (width 0.25) (layer F.Cu) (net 16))
 (segment (start 159.555 108.8323) (end 158.623 108.8323) (width 0.25) (layer F.Cu) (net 16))
 (segment (start 157.31 109.22) (end 158.2353 109.22) (width 0.25) (layer F.Cu) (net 16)))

